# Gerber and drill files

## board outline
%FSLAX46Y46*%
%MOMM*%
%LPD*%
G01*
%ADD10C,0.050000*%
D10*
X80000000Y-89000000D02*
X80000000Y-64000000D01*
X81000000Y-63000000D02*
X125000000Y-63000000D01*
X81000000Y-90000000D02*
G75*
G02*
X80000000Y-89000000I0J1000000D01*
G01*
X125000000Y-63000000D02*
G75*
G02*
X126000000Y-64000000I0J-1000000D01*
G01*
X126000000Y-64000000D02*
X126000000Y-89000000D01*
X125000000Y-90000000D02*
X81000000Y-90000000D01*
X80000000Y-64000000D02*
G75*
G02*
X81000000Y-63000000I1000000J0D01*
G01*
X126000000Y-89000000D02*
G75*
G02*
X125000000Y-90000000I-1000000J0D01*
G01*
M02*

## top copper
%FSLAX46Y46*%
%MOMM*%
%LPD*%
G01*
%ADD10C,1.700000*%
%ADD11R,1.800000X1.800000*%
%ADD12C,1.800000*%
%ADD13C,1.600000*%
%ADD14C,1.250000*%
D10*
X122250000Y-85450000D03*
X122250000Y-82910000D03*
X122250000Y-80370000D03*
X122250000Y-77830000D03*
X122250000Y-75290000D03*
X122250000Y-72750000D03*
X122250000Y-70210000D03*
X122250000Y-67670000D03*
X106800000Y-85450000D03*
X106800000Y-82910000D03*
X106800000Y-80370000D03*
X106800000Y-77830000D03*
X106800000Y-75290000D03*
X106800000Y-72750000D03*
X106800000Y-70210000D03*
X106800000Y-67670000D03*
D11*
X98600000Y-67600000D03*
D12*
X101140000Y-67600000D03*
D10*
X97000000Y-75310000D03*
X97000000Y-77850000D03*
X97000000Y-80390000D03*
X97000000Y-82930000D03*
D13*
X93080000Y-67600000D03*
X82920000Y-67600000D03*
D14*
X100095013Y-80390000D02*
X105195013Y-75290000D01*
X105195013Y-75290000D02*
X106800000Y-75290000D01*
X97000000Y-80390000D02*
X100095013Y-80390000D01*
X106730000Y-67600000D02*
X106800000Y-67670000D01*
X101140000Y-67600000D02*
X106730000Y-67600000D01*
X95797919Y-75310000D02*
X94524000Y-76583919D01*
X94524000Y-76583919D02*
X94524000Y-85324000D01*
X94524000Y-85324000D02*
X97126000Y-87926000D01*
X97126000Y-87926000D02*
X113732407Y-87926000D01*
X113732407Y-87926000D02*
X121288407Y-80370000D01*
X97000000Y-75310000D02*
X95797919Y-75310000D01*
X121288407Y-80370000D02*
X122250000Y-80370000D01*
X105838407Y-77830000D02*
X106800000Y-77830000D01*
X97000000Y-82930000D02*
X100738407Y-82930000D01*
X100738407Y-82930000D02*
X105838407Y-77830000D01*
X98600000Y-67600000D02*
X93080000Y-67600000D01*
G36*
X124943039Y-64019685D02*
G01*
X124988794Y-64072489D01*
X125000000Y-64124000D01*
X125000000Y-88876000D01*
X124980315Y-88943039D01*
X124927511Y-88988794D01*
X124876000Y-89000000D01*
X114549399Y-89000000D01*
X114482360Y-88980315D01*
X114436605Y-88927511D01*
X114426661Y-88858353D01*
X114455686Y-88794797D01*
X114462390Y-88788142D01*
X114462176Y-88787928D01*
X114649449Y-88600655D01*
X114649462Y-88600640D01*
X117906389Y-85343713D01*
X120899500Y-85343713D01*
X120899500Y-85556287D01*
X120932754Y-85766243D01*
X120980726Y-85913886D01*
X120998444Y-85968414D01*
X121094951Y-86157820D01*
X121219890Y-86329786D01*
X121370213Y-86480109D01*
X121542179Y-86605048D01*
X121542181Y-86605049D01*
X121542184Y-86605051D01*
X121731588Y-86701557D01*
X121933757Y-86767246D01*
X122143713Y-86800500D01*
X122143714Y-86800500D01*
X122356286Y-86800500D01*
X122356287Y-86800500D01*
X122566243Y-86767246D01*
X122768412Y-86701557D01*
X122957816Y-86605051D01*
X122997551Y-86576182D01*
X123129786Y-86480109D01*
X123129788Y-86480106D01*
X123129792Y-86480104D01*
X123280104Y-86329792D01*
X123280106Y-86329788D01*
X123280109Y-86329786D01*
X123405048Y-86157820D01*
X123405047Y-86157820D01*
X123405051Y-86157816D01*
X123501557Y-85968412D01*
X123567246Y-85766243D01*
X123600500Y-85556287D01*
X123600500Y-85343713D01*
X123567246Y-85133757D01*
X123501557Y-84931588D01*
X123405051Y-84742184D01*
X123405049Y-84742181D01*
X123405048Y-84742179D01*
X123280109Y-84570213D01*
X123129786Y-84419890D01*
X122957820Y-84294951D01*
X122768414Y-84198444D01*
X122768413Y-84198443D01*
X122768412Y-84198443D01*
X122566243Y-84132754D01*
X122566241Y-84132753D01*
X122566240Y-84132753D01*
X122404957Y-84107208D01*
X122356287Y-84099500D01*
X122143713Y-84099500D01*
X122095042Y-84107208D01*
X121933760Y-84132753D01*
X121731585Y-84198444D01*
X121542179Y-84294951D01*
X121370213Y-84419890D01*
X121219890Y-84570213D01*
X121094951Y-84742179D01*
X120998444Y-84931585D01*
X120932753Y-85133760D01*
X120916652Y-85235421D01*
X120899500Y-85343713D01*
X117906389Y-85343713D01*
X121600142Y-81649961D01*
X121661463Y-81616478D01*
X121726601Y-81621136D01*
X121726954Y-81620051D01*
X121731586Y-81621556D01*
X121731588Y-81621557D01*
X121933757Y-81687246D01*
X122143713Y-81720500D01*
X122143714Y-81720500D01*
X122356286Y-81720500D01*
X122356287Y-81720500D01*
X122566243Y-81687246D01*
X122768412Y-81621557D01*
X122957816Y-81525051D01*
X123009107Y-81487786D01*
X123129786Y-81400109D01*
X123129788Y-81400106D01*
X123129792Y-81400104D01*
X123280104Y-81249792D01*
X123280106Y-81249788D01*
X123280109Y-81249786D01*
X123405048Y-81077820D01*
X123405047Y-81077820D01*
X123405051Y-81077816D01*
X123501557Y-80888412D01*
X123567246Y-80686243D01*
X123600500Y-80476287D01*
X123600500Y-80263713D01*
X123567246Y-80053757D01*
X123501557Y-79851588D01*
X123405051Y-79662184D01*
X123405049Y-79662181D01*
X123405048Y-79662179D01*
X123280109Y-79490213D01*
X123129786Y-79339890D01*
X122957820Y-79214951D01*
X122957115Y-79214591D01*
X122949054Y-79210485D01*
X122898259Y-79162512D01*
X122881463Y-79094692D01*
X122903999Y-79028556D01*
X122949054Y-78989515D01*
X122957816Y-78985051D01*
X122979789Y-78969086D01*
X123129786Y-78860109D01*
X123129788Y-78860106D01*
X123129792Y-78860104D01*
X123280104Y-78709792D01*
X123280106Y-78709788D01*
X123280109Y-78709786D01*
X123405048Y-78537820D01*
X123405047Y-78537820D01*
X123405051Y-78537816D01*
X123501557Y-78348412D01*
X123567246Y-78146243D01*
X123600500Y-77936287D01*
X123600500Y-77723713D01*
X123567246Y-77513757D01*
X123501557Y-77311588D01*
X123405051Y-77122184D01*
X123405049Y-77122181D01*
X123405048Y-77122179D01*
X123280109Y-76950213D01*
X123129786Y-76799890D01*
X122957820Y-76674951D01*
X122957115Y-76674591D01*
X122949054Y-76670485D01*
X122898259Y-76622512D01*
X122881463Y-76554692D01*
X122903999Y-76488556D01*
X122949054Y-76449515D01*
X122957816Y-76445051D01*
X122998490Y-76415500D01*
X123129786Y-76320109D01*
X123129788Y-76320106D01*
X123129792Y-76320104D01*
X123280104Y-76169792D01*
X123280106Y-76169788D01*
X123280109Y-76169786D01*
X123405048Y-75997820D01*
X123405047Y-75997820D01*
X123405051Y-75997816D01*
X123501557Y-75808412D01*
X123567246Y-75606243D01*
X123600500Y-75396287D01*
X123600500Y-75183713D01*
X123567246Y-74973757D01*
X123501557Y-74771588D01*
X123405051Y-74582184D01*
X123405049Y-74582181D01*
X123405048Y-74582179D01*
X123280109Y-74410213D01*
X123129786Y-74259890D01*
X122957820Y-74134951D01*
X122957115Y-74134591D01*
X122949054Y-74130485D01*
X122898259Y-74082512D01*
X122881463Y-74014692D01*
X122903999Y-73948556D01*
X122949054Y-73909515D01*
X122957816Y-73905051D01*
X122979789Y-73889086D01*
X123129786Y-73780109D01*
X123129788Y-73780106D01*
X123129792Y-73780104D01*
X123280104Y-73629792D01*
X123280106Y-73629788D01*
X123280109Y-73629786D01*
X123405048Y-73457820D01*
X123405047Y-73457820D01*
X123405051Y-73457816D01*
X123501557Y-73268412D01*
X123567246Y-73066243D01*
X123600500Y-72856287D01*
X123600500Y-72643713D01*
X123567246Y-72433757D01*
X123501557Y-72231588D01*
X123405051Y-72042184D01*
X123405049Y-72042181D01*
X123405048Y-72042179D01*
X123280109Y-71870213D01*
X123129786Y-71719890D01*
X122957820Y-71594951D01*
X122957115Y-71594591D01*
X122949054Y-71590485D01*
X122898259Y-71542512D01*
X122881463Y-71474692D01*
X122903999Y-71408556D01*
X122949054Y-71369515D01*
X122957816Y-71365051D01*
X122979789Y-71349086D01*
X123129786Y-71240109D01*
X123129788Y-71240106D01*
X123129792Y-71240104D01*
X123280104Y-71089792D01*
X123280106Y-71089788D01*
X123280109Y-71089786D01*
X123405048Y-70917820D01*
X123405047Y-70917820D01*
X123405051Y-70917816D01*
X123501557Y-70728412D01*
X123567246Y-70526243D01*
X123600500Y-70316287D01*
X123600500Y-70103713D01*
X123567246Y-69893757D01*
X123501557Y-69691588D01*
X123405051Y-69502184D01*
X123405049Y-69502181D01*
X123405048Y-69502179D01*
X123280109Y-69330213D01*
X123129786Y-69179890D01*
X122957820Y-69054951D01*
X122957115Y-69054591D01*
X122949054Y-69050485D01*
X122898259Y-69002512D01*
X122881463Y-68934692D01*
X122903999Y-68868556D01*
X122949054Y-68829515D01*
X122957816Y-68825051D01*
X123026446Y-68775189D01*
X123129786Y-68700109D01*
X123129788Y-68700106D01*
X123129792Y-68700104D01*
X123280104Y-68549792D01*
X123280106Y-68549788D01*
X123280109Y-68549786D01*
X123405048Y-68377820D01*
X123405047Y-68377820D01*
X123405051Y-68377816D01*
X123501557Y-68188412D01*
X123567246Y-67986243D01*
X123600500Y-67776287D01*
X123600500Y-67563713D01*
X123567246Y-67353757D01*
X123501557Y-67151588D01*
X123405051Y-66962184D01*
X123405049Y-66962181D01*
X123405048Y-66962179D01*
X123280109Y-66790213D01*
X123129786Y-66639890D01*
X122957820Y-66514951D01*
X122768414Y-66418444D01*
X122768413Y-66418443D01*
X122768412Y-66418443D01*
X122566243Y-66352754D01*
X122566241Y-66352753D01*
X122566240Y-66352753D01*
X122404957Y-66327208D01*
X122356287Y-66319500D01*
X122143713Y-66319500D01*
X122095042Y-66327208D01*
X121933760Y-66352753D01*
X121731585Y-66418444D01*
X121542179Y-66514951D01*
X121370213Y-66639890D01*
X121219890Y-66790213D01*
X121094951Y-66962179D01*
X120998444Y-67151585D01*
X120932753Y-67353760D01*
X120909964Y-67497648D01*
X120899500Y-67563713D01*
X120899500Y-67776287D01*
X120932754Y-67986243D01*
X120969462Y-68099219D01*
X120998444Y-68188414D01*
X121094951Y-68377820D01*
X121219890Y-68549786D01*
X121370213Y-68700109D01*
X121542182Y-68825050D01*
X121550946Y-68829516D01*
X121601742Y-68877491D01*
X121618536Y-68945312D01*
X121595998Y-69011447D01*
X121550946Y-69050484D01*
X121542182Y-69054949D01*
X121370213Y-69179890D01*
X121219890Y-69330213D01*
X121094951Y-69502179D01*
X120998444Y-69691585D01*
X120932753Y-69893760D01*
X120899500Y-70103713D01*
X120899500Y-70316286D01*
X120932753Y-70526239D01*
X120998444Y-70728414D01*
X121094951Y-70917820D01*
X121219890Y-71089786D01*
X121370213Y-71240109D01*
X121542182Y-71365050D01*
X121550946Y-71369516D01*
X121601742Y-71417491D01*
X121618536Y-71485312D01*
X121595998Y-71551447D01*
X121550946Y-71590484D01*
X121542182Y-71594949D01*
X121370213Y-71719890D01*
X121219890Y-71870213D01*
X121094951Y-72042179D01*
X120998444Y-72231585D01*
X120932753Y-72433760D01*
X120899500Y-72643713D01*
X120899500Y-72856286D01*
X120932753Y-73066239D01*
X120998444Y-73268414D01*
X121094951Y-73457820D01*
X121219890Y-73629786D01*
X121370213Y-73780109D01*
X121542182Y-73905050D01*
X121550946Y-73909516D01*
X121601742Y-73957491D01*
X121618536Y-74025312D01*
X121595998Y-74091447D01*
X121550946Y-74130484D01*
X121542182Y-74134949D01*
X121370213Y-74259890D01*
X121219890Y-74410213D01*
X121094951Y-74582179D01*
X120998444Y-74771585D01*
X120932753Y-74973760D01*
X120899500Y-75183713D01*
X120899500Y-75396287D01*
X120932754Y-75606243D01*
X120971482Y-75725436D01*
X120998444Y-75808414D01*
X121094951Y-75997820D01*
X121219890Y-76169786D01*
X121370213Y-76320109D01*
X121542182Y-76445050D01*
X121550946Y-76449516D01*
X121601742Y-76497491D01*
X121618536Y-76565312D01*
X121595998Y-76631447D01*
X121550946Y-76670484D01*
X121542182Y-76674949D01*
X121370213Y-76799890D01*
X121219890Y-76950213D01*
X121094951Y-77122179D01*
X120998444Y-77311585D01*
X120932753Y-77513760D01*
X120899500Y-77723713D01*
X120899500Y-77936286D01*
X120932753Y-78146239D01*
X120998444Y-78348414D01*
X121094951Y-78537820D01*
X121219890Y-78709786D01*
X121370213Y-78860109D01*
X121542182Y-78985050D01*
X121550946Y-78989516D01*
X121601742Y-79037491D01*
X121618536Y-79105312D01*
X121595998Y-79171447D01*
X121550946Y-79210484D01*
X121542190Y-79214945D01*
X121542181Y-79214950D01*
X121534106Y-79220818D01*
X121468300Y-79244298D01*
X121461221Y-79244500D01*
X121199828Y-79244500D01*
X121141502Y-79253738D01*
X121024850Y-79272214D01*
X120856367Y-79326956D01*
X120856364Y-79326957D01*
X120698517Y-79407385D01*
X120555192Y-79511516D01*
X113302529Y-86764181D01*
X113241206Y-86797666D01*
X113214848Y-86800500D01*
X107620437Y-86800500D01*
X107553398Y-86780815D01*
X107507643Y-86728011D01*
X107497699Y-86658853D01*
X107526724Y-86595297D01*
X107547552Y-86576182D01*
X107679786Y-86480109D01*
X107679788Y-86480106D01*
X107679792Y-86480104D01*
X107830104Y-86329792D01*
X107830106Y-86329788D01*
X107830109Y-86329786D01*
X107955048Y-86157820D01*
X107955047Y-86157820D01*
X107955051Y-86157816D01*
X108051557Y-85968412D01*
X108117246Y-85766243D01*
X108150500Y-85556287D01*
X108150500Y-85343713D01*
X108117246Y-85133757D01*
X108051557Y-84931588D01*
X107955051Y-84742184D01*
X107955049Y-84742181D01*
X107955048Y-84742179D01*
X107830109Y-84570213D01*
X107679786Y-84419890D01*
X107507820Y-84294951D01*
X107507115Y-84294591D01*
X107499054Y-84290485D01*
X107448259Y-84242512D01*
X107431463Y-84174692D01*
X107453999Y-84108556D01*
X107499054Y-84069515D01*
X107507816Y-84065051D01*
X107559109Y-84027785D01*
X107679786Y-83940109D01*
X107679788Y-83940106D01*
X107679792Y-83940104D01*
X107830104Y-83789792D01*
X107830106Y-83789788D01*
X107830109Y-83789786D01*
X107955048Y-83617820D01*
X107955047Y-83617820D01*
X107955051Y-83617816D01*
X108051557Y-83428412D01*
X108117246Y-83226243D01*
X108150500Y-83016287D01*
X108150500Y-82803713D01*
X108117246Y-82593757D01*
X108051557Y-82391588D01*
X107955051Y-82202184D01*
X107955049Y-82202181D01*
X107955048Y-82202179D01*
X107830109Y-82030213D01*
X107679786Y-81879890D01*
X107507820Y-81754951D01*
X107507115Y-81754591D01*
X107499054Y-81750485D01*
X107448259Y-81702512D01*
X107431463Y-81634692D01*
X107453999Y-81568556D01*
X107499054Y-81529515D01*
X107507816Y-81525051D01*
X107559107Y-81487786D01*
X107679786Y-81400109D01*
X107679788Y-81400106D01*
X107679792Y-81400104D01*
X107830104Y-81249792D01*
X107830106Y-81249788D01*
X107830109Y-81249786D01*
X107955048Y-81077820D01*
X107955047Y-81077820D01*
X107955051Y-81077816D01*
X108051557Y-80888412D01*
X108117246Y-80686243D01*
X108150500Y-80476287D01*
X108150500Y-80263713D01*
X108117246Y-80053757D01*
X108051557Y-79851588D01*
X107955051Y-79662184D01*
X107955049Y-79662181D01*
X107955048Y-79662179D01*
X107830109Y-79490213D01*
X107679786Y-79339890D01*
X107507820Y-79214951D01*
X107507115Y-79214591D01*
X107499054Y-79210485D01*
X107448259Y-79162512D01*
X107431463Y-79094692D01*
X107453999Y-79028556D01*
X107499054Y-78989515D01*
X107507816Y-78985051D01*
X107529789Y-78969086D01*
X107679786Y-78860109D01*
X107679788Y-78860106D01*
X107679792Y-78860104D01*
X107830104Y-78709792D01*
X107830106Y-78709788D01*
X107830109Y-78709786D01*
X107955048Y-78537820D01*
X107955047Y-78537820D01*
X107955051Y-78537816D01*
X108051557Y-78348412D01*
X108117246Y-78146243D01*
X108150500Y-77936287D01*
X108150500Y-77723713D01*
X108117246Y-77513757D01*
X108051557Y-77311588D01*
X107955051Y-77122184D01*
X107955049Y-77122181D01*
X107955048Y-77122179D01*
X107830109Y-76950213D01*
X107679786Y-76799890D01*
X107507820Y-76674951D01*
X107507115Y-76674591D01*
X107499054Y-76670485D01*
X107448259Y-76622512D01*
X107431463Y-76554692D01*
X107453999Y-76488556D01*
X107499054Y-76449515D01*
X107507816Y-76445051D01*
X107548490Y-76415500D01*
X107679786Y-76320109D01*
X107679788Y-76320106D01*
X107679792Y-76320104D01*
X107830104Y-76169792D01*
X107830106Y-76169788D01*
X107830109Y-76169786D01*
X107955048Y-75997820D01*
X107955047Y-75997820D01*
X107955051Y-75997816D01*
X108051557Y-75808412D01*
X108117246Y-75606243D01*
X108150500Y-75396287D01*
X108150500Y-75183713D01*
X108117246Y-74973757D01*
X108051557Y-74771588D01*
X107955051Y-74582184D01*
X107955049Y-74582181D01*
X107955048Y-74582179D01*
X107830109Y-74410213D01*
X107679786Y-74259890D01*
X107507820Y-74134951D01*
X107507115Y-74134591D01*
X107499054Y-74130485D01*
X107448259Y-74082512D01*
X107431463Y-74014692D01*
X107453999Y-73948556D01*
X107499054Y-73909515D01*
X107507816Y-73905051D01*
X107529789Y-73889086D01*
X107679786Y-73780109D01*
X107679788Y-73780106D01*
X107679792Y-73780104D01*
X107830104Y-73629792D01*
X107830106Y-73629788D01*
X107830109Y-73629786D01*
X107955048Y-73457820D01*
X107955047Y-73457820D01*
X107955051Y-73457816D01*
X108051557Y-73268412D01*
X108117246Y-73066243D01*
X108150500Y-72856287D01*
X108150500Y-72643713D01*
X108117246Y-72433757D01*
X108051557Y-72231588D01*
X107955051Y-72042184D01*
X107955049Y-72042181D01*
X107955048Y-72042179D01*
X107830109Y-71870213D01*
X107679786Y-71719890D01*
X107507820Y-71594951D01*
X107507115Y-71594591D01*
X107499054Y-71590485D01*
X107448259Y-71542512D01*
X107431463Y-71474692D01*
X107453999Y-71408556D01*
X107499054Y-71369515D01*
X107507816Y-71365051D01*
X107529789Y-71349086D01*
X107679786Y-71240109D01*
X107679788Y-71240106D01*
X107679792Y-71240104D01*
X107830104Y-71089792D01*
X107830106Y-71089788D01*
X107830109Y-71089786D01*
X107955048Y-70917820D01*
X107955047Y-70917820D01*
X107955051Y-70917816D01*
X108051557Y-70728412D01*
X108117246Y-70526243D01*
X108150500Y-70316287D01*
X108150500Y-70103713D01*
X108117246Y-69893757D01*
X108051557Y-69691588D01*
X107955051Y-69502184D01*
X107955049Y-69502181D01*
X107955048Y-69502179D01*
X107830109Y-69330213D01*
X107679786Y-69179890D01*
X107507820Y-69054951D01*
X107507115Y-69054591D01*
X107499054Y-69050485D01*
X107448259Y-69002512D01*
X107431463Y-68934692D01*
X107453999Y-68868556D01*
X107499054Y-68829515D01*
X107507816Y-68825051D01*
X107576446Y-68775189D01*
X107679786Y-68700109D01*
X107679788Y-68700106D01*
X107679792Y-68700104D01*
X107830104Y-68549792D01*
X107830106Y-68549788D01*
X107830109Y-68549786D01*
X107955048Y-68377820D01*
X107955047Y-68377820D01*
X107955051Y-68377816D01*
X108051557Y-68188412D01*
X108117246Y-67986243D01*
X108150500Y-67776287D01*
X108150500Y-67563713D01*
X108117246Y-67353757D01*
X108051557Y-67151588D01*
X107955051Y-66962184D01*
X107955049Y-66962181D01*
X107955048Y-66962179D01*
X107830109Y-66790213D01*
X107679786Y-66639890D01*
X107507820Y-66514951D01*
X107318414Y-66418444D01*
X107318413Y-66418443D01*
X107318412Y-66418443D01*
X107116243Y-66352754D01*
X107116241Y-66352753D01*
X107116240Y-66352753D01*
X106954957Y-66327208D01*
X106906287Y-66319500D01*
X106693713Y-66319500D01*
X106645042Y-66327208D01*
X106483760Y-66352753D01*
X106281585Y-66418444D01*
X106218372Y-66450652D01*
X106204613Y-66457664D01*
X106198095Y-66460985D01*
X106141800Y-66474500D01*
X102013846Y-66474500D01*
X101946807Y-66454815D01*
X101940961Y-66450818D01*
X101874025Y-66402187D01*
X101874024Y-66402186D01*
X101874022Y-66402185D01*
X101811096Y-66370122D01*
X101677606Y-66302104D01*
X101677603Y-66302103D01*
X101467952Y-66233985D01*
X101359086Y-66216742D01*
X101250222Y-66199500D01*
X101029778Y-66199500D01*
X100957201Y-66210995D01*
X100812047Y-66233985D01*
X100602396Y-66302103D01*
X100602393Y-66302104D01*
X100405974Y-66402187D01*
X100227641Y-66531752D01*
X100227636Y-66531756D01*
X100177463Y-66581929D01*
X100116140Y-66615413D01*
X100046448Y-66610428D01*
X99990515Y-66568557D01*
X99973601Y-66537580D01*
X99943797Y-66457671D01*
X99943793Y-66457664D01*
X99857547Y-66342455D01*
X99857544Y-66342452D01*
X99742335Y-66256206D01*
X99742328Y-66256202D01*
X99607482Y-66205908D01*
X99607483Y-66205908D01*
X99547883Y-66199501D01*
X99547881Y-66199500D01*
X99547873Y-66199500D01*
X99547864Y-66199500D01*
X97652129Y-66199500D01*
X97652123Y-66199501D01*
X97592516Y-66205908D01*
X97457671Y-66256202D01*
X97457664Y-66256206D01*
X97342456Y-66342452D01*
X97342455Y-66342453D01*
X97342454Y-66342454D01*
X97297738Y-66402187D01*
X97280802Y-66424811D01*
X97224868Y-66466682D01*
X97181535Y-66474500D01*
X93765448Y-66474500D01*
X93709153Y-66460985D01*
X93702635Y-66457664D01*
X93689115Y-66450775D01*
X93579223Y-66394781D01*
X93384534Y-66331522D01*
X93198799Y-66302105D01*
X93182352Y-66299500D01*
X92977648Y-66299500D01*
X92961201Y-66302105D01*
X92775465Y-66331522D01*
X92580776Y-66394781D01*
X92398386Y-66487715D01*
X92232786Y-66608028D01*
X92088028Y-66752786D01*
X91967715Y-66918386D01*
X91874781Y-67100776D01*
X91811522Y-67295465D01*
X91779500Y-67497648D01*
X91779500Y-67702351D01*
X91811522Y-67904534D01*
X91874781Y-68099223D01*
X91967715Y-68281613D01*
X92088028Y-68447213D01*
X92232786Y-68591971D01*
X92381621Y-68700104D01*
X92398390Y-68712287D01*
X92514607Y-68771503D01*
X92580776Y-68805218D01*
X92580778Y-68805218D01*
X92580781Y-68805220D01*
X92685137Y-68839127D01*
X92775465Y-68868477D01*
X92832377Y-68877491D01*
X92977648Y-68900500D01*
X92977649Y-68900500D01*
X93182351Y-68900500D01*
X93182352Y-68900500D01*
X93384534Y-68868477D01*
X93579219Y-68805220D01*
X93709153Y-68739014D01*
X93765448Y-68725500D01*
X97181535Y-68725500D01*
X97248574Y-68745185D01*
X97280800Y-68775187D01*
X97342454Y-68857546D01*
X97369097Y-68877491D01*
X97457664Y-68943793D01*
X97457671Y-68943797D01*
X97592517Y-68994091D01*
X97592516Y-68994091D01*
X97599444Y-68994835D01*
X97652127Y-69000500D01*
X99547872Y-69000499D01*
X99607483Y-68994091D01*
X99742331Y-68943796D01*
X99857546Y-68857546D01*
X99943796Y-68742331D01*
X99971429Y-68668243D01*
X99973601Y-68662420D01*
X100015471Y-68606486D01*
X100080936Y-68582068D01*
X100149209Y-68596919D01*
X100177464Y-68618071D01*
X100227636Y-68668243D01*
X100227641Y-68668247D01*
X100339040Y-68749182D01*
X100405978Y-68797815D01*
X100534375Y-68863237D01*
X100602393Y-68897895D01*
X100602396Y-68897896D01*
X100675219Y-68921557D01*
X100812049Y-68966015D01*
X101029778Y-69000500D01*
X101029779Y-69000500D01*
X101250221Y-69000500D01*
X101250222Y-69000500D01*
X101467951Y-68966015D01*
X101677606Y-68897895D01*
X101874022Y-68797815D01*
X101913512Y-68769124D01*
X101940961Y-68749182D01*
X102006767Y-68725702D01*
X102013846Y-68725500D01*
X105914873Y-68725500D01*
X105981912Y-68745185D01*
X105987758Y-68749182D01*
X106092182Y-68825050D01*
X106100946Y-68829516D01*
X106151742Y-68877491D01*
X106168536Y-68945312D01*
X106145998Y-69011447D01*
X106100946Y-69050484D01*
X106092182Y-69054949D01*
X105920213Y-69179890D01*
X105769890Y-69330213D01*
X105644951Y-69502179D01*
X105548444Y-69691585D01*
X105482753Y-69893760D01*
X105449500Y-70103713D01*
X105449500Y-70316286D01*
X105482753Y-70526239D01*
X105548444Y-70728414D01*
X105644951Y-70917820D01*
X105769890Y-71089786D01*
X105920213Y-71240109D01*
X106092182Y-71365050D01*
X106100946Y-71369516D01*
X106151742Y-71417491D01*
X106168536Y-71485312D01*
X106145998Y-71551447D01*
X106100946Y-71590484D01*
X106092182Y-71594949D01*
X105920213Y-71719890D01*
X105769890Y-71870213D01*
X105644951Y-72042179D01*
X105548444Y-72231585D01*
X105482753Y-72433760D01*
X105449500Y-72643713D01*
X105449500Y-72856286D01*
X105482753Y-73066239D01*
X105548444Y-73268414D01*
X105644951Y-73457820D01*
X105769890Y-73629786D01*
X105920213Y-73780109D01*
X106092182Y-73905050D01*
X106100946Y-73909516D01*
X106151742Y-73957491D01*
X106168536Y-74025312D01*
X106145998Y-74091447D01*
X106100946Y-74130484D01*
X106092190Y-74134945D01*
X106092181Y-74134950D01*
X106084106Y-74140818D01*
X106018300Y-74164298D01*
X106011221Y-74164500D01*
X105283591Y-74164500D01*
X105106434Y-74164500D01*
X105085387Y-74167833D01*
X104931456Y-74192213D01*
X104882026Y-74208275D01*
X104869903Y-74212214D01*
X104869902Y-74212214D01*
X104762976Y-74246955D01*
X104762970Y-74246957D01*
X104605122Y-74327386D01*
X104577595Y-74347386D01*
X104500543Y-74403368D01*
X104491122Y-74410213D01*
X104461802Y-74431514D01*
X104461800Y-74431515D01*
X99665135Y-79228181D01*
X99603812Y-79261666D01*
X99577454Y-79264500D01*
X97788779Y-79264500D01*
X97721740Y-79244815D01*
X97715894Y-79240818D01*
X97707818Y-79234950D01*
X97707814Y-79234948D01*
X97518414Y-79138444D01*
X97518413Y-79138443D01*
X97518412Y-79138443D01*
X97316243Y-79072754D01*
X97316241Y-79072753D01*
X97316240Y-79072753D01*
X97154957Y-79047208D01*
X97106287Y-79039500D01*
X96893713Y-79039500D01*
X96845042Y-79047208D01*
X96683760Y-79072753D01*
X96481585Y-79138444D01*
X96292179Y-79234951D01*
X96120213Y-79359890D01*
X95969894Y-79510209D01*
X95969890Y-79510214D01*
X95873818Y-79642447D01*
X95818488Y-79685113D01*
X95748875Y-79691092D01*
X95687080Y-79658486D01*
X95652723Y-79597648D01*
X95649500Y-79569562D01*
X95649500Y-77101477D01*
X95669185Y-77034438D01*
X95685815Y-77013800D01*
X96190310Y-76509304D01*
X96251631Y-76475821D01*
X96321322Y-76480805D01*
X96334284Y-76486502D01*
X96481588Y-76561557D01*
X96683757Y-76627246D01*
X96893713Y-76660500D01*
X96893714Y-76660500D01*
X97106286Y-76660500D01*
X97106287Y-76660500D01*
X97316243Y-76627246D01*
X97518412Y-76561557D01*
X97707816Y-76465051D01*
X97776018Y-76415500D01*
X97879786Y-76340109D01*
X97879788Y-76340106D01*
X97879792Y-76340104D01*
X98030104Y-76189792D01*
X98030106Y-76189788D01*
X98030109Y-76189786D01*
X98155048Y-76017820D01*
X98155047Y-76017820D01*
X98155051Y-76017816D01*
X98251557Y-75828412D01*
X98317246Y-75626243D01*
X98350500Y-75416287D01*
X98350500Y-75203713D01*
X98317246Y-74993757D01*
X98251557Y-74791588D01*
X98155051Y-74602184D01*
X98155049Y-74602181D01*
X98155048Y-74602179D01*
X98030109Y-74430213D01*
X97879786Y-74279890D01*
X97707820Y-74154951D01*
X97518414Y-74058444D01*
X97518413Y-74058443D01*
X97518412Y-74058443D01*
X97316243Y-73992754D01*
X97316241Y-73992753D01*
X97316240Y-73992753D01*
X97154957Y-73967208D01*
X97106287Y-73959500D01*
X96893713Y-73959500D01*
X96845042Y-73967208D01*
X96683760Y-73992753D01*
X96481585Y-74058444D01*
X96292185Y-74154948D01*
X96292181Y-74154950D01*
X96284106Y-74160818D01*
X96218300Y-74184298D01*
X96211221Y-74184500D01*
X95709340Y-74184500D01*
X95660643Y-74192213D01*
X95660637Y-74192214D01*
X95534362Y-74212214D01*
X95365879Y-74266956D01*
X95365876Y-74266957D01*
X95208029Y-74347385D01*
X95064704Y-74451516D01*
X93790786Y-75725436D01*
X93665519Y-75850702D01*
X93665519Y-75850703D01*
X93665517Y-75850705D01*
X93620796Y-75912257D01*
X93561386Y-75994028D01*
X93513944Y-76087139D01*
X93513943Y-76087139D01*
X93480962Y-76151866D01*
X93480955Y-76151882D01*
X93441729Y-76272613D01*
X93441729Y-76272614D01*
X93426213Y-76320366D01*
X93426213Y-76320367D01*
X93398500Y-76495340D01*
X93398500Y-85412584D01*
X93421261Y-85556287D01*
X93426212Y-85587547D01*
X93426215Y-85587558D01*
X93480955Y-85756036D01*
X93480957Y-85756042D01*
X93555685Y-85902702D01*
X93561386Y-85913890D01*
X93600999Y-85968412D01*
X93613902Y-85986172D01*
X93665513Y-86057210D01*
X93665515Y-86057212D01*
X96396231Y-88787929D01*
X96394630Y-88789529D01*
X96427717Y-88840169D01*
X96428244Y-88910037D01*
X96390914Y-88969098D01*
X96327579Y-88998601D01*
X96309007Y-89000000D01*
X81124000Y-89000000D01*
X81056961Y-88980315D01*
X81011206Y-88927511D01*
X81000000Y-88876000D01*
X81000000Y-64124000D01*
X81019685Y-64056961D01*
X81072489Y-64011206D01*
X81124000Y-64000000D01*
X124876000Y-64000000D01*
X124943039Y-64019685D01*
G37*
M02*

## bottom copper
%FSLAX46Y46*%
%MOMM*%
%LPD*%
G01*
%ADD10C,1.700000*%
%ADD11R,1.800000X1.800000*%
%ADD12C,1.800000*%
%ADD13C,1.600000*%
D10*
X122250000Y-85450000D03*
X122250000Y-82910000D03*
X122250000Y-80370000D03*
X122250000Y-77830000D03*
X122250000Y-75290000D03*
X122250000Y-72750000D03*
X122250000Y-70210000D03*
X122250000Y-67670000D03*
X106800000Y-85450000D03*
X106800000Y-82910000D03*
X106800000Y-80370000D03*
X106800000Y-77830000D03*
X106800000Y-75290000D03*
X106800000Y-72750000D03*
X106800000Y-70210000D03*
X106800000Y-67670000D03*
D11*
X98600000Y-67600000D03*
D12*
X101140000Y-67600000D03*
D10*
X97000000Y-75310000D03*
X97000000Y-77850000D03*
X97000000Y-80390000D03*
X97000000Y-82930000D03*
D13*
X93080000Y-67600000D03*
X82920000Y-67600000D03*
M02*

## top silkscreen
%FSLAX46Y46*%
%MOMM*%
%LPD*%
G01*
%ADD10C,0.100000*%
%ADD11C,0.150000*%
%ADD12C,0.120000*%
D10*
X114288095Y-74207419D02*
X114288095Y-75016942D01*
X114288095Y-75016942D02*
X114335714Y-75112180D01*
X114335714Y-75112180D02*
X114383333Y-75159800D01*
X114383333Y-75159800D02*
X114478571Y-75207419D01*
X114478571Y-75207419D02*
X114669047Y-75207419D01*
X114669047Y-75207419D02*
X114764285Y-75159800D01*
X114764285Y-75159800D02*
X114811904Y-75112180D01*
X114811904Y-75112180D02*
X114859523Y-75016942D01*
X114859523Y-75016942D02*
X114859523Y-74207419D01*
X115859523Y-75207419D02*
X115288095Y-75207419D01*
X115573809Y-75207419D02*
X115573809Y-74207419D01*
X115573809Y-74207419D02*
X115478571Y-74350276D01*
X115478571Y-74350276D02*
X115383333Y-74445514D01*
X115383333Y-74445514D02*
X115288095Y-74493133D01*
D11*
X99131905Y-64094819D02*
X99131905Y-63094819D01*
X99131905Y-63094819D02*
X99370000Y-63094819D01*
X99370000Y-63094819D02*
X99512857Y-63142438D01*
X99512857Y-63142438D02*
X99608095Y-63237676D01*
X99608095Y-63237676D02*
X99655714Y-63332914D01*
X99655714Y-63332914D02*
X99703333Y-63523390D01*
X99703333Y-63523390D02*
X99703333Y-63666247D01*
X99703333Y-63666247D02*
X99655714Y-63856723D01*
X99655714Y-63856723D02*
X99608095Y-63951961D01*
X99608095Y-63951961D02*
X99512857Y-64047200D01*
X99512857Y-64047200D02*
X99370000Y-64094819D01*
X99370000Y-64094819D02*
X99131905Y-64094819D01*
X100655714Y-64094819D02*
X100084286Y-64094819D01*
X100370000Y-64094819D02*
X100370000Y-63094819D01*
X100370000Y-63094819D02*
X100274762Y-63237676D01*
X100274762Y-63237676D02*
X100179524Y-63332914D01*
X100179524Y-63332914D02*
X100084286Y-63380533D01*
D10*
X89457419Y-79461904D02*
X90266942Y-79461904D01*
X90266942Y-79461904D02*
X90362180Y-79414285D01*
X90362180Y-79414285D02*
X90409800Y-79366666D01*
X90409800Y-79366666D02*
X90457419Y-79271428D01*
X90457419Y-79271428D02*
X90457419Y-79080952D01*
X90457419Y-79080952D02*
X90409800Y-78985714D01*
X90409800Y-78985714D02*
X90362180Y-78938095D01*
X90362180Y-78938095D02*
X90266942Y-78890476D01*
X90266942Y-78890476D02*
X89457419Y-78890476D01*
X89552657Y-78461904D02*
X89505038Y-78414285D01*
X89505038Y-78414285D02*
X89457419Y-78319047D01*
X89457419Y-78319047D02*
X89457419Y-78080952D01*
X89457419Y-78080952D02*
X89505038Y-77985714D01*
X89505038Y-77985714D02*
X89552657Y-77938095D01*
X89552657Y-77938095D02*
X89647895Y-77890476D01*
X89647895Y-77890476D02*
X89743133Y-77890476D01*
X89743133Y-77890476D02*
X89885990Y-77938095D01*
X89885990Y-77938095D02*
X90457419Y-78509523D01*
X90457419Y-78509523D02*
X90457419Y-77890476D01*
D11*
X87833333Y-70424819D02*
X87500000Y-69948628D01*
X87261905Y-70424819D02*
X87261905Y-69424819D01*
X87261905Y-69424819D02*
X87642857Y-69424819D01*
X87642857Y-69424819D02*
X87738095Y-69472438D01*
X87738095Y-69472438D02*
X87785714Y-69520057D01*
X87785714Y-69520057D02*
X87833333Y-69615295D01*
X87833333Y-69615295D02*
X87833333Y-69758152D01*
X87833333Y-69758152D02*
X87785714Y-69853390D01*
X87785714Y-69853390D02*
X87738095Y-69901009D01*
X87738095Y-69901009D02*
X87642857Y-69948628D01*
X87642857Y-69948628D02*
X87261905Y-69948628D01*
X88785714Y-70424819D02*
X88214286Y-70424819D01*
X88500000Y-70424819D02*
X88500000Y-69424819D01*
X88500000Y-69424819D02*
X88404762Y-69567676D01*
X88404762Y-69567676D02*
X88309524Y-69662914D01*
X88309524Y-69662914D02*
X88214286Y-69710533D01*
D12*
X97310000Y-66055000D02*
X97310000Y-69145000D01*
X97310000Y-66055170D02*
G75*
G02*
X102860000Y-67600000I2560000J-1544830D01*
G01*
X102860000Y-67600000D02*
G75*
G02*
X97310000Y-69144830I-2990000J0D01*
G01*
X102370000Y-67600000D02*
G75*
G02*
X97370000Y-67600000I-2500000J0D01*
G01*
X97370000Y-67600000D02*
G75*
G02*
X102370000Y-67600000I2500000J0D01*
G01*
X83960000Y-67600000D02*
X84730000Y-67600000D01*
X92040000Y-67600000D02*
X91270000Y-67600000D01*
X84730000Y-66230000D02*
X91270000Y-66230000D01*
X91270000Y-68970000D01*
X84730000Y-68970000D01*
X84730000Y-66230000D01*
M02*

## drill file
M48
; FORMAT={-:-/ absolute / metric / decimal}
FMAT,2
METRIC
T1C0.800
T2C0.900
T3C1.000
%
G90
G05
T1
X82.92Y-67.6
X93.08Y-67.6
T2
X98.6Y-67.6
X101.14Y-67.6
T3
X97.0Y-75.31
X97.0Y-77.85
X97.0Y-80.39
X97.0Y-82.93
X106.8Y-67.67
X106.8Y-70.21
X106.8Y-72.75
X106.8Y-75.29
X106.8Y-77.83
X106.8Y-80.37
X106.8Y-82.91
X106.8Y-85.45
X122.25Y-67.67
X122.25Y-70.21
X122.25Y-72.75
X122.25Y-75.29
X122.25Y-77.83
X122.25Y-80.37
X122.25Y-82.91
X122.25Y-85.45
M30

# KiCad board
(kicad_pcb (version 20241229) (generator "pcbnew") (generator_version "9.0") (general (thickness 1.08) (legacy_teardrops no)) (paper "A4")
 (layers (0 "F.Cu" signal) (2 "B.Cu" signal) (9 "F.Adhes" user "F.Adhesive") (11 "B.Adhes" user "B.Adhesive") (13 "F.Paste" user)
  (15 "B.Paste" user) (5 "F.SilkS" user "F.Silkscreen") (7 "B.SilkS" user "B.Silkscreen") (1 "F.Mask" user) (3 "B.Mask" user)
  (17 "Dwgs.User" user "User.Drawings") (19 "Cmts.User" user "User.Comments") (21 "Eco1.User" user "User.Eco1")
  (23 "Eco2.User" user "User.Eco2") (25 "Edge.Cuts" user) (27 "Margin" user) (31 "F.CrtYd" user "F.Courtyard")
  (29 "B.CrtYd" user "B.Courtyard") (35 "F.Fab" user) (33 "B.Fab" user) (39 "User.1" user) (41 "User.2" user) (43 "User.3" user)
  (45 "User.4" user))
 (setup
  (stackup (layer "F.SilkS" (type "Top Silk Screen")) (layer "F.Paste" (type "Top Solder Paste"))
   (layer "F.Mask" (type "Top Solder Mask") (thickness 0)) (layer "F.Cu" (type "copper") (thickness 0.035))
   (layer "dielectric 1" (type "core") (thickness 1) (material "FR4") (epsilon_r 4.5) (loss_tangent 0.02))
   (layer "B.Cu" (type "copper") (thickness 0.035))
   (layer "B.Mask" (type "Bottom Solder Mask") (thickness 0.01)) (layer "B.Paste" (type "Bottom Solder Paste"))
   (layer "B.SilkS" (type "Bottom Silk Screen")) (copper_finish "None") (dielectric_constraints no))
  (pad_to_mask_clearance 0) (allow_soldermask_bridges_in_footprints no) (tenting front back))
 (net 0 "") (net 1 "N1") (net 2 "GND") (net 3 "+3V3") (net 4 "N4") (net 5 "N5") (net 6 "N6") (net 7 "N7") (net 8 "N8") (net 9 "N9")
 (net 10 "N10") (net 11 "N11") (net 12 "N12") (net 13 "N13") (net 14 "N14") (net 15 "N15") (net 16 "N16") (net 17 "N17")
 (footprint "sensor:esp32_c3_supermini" (layer "F.Cu") (at 115.05 75.25)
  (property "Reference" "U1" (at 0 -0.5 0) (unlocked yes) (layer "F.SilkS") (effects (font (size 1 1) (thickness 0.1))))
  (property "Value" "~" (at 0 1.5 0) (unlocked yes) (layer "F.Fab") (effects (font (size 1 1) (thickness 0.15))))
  (pad "1" thru_hole circle (at 7.2 10.2) (size 1.7 1.7) (drill 1) (layers "*.Cu" "*.Mask") (remove_unused_layers no) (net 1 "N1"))
  (pad "2" thru_hole circle (at 7.2 7.66) (size 1.7 1.7) (drill 1) (layers "*.Cu" "*.Mask") (remove_unused_layers no) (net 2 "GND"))
  (pad "3" thru_hole circle (at 7.2 5.12) (size 1.7 1.7) (drill 1) (layers "*.Cu" "*.Mask") (remove_unused_layers no) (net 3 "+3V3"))
  (pad "4" thru_hole circle (at 7.2 2.58) (size 1.7 1.7) (drill 1) (layers "*.Cu" "*.Mask") (remove_unused_layers no) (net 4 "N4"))
  (pad "5" thru_hole circle (at 7.2 0.04) (size 1.7 1.7) (drill 1) (layers "*.Cu" "*.Mask") (remove_unused_layers no) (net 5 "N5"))
  (pad "6" thru_hole circle (at 7.2 -2.5) (size 1.7 1.7) (drill 1) (layers "*.Cu" "*.Mask") (remove_unused_layers no) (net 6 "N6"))
  (pad "7" thru_hole circle (at 7.2 -5.04) (size 1.7 1.7) (drill 1) (layers "*.Cu" "*.Mask") (remove_unused_layers no) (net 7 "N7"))
  (pad "8" thru_hole circle (at 7.2 -7.58) (size 1.7 1.7) (drill 1) (layers "*.Cu" "*.Mask") (remove_unused_layers no) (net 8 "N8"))
  (pad "9" thru_hole circle (at -8.25 10.2) (size 1.7 1.7) (drill 1) (layers "*.Cu" "*.Mask") (remove_unused_layers no) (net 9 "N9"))
  (pad "10" thru_hole circle (at -8.25 7.66) (size 1.7 1.7) (drill 1) (layers "*.Cu" "*.Mask") (remove_unused_layers no) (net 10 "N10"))
  (pad "11" thru_hole circle (at -8.25 5.12) (size 1.7 1.7) (drill 1) (layers "*.Cu" "*.Mask") (remove_unused_layers no) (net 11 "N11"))
  (pad "12" thru_hole circle (at -8.25 2.58) (size 1.7 1.7) (drill 1) (layers "*.Cu" "*.Mask") (remove_unused_layers no) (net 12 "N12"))
  (pad "13" thru_hole circle (at -8.25 0.04) (size 1.7 1.7) (drill 1) (layers "*.Cu" "*.Mask") (remove_unused_layers no) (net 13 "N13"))
  (pad "14" thru_hole circle (at -8.25 -2.5) (size 1.7 1.7) (drill 1) (layers "*.Cu" "*.Mask") (remove_unused_layers no) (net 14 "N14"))
  (pad "15" thru_hole circle (at -8.25 -5.04) (size 1.7 1.7) (drill 1) (layers "*.Cu" "*.Mask") (remove_unused_layers no) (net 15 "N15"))
  (pad "16" thru_hole circle (at -8.25 -7.58) (size 1.7 1.7) (drill 1) (layers "*.Cu" "*.Mask") (remove_unused_layers no) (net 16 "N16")))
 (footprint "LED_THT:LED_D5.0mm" (layer "F.Cu") (at 98.6 67.6)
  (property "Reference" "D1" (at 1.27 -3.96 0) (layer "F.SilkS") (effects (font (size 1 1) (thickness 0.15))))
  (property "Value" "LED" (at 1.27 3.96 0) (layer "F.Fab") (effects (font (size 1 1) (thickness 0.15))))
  (fp_line (start -1.29 -1.545) (end -1.29 1.545) (stroke (width 0.12) (type solid)) (layer "F.SilkS"))
  (fp_arc (start -1.29 -1.54483) (mid 2.071779 -2.880495) (end 4.26 0) (stroke (width 0.12) (type solid)) (layer "F.SilkS"))
  (fp_arc (start 4.26 0) (mid 2.071779 2.880495) (end -1.29 1.54483) (stroke (width 0.12) (type solid)) (layer "F.SilkS"))
  (fp_circle (center 1.27 0) (end 3.77 0) (stroke (width 0.12) (type solid)) (fill no) (layer "F.SilkS"))
  (pad "1" thru_hole rect (at 0 0) (size 1.8 1.8) (drill 0.9) (layers "*.Cu" "*.Mask") (remove_unused_layers no) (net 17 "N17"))
  (pad "2" thru_hole circle (at 2.54 0) (size 1.8 1.8) (drill 0.9) (layers "*.Cu" "*.Mask") (remove_unused_layers no) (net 16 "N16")))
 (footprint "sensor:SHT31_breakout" (layer "F.Cu") (at 90.5 78.7 90)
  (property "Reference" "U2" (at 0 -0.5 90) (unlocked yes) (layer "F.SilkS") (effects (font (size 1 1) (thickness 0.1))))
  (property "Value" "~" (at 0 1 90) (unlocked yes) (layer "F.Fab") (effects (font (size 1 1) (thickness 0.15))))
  (pad "1" thru_hole circle (at 3.39 6.5) (size 1.7 1.7) (drill 1) (layers "*.Cu" "*.Mask") (remove_unused_layers no) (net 3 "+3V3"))
  (pad "2" thru_hole circle (at 0.85 6.5) (size 1.7 1.7) (drill 1) (layers "*.Cu" "*.Mask") (remove_unused_layers no) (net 2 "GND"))
  (pad "3" thru_hole circle (at -1.69 6.5) (size 1.7 1.7) (drill 1) (layers "*.Cu" "*.Mask") (remove_unused_layers no) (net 13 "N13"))
  (pad "4" thru_hole circle (at -4.23 6.5) (size 1.7 1.7) (drill 1) (layers "*.Cu" "*.Mask") (remove_unused_layers no) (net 12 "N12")))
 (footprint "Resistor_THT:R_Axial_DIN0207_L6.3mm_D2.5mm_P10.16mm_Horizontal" (layer "F.Cu") (at 93.08 67.6 180)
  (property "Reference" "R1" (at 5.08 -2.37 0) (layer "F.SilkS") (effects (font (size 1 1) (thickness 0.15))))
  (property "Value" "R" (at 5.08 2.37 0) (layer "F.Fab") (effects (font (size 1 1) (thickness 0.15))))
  (fp_line (start 9.12 0) (end 8.35 0) (stroke (width 0.12) (type solid)) (layer "F.SilkS"))
  (fp_line (start 1.04 0) (end 1.81 0) (stroke (width 0.12) (type solid)) (layer "F.SilkS"))
  (fp_rect (start 1.81 -1.37) (end 8.35 1.37) (stroke (width 0.12) (type solid)) (fill no) (layer "F.SilkS"))
  (pad "1" thru_hole circle (at 0 0 180) (size 1.6 1.6) (drill 0.8) (layers "*.Cu" "*.Mask") (remove_unused_layers no) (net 17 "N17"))
  (pad "2" thru_hole circle (at 10.16 0 180) (size 1.6 1.6) (drill 0.8) (layers "*.Cu" "*.Mask") (remove_unused_layers no) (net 2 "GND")))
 (gr_line (start 80 89) (end 80 64) (stroke (width 0.05) (type default)) (layer "Edge.Cuts"))
 (gr_line (start 81 63) (end 125 63) (stroke (width 0.05) (type default)) (layer "Edge.Cuts"))
 (gr_arc (start 81 90) (mid 80.292893 89.707107) (end 80 89) (stroke (width 0.05) (type default)) (layer "Edge.Cuts"))
 (gr_arc (start 125 63) (mid 125.707107 63.292893) (end 126 64) (stroke (width 0.05) (type default)) (layer "Edge.Cuts"))
 (gr_line (start 126 64) (end 126 89) (stroke (width 0.05) (type default)) (layer "Edge.Cuts"))
 (gr_line (start 125 90) (end 81 90) (stroke (width 0.05) (type default)) (layer "Edge.Cuts"))
 (gr_arc (start 80 64) (mid 80.292893 63.292893) (end 81 63) (stroke (width 0.05) (type default)) (layer "Edge.Cuts"))
 (gr_arc (start 126 89) (mid 125.707107 89.707107) (end 125 90) (stroke (width 0.05) (type default)) (layer "Edge.Cuts"))
 (segment (start 100.095013 80.39) (end 105.195013 75.29) (width 1.25) (layer "F.Cu") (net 13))
 (segment (start 105.195013 75.29) (end 106.8 75.29) (width 1.25) (layer "F.Cu") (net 13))
 (segment (start 97 80.39) (end 100.095013 80.39) (width 1.25) (layer "F.Cu") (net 13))
 (segment (start 106.73 67.6) (end 106.8 67.67) (width 1.25) (layer "F.Cu") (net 16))
 (segment (start 101.14 67.6) (end 106.73 67.6) (width 1.25) (layer "F.Cu") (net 16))
 (segment (start 95.797919 75.31) (end 94.524 76.583919) (width 1.25) (layer "F.Cu") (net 3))
 (segment (start 94.524 76.583919) (end 94.524 85.324) (width 1.25) (layer "F.Cu") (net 3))
 (segment (start 94.524 85.324) (end 97.126 87.926) (width 1.25) (layer "F.Cu") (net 3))
 (segment (start 97.126 87.926) (end 113.732407 87.926) (width 1.25) (layer "F.Cu") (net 3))
 (segment (start 113.732407 87.926) (end 121.288407 80.37) (width 1.25) (layer "F.Cu") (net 3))
 (segment (start 97 75.31) (end 95.797919 75.31) (width 1.25) (layer "F.Cu") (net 3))
 (segment (start 121.288407 80.37) (end 122.25 80.37) (width 1.25) (layer "F.Cu") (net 3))
 (segment (start 105.838407 77.83) (end 106.8 77.83) (width 1.25) (layer "F.Cu") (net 12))
 (segment (start 97 82.93) (end 100.738407 82.93) (width 1.25) (layer "F.Cu") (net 12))
 (segment (start 100.738407 82.93) (end 105.838407 77.83) (width 1.25) (layer "F.Cu") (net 12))
 (segment (start 98.6 67.6) (end 93.08 67.6) (width 1.25) (layer "F.Cu") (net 17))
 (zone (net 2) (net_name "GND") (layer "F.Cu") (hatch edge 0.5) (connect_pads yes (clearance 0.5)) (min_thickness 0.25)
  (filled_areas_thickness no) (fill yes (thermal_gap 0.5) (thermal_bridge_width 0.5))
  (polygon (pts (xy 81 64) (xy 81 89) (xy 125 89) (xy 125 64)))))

